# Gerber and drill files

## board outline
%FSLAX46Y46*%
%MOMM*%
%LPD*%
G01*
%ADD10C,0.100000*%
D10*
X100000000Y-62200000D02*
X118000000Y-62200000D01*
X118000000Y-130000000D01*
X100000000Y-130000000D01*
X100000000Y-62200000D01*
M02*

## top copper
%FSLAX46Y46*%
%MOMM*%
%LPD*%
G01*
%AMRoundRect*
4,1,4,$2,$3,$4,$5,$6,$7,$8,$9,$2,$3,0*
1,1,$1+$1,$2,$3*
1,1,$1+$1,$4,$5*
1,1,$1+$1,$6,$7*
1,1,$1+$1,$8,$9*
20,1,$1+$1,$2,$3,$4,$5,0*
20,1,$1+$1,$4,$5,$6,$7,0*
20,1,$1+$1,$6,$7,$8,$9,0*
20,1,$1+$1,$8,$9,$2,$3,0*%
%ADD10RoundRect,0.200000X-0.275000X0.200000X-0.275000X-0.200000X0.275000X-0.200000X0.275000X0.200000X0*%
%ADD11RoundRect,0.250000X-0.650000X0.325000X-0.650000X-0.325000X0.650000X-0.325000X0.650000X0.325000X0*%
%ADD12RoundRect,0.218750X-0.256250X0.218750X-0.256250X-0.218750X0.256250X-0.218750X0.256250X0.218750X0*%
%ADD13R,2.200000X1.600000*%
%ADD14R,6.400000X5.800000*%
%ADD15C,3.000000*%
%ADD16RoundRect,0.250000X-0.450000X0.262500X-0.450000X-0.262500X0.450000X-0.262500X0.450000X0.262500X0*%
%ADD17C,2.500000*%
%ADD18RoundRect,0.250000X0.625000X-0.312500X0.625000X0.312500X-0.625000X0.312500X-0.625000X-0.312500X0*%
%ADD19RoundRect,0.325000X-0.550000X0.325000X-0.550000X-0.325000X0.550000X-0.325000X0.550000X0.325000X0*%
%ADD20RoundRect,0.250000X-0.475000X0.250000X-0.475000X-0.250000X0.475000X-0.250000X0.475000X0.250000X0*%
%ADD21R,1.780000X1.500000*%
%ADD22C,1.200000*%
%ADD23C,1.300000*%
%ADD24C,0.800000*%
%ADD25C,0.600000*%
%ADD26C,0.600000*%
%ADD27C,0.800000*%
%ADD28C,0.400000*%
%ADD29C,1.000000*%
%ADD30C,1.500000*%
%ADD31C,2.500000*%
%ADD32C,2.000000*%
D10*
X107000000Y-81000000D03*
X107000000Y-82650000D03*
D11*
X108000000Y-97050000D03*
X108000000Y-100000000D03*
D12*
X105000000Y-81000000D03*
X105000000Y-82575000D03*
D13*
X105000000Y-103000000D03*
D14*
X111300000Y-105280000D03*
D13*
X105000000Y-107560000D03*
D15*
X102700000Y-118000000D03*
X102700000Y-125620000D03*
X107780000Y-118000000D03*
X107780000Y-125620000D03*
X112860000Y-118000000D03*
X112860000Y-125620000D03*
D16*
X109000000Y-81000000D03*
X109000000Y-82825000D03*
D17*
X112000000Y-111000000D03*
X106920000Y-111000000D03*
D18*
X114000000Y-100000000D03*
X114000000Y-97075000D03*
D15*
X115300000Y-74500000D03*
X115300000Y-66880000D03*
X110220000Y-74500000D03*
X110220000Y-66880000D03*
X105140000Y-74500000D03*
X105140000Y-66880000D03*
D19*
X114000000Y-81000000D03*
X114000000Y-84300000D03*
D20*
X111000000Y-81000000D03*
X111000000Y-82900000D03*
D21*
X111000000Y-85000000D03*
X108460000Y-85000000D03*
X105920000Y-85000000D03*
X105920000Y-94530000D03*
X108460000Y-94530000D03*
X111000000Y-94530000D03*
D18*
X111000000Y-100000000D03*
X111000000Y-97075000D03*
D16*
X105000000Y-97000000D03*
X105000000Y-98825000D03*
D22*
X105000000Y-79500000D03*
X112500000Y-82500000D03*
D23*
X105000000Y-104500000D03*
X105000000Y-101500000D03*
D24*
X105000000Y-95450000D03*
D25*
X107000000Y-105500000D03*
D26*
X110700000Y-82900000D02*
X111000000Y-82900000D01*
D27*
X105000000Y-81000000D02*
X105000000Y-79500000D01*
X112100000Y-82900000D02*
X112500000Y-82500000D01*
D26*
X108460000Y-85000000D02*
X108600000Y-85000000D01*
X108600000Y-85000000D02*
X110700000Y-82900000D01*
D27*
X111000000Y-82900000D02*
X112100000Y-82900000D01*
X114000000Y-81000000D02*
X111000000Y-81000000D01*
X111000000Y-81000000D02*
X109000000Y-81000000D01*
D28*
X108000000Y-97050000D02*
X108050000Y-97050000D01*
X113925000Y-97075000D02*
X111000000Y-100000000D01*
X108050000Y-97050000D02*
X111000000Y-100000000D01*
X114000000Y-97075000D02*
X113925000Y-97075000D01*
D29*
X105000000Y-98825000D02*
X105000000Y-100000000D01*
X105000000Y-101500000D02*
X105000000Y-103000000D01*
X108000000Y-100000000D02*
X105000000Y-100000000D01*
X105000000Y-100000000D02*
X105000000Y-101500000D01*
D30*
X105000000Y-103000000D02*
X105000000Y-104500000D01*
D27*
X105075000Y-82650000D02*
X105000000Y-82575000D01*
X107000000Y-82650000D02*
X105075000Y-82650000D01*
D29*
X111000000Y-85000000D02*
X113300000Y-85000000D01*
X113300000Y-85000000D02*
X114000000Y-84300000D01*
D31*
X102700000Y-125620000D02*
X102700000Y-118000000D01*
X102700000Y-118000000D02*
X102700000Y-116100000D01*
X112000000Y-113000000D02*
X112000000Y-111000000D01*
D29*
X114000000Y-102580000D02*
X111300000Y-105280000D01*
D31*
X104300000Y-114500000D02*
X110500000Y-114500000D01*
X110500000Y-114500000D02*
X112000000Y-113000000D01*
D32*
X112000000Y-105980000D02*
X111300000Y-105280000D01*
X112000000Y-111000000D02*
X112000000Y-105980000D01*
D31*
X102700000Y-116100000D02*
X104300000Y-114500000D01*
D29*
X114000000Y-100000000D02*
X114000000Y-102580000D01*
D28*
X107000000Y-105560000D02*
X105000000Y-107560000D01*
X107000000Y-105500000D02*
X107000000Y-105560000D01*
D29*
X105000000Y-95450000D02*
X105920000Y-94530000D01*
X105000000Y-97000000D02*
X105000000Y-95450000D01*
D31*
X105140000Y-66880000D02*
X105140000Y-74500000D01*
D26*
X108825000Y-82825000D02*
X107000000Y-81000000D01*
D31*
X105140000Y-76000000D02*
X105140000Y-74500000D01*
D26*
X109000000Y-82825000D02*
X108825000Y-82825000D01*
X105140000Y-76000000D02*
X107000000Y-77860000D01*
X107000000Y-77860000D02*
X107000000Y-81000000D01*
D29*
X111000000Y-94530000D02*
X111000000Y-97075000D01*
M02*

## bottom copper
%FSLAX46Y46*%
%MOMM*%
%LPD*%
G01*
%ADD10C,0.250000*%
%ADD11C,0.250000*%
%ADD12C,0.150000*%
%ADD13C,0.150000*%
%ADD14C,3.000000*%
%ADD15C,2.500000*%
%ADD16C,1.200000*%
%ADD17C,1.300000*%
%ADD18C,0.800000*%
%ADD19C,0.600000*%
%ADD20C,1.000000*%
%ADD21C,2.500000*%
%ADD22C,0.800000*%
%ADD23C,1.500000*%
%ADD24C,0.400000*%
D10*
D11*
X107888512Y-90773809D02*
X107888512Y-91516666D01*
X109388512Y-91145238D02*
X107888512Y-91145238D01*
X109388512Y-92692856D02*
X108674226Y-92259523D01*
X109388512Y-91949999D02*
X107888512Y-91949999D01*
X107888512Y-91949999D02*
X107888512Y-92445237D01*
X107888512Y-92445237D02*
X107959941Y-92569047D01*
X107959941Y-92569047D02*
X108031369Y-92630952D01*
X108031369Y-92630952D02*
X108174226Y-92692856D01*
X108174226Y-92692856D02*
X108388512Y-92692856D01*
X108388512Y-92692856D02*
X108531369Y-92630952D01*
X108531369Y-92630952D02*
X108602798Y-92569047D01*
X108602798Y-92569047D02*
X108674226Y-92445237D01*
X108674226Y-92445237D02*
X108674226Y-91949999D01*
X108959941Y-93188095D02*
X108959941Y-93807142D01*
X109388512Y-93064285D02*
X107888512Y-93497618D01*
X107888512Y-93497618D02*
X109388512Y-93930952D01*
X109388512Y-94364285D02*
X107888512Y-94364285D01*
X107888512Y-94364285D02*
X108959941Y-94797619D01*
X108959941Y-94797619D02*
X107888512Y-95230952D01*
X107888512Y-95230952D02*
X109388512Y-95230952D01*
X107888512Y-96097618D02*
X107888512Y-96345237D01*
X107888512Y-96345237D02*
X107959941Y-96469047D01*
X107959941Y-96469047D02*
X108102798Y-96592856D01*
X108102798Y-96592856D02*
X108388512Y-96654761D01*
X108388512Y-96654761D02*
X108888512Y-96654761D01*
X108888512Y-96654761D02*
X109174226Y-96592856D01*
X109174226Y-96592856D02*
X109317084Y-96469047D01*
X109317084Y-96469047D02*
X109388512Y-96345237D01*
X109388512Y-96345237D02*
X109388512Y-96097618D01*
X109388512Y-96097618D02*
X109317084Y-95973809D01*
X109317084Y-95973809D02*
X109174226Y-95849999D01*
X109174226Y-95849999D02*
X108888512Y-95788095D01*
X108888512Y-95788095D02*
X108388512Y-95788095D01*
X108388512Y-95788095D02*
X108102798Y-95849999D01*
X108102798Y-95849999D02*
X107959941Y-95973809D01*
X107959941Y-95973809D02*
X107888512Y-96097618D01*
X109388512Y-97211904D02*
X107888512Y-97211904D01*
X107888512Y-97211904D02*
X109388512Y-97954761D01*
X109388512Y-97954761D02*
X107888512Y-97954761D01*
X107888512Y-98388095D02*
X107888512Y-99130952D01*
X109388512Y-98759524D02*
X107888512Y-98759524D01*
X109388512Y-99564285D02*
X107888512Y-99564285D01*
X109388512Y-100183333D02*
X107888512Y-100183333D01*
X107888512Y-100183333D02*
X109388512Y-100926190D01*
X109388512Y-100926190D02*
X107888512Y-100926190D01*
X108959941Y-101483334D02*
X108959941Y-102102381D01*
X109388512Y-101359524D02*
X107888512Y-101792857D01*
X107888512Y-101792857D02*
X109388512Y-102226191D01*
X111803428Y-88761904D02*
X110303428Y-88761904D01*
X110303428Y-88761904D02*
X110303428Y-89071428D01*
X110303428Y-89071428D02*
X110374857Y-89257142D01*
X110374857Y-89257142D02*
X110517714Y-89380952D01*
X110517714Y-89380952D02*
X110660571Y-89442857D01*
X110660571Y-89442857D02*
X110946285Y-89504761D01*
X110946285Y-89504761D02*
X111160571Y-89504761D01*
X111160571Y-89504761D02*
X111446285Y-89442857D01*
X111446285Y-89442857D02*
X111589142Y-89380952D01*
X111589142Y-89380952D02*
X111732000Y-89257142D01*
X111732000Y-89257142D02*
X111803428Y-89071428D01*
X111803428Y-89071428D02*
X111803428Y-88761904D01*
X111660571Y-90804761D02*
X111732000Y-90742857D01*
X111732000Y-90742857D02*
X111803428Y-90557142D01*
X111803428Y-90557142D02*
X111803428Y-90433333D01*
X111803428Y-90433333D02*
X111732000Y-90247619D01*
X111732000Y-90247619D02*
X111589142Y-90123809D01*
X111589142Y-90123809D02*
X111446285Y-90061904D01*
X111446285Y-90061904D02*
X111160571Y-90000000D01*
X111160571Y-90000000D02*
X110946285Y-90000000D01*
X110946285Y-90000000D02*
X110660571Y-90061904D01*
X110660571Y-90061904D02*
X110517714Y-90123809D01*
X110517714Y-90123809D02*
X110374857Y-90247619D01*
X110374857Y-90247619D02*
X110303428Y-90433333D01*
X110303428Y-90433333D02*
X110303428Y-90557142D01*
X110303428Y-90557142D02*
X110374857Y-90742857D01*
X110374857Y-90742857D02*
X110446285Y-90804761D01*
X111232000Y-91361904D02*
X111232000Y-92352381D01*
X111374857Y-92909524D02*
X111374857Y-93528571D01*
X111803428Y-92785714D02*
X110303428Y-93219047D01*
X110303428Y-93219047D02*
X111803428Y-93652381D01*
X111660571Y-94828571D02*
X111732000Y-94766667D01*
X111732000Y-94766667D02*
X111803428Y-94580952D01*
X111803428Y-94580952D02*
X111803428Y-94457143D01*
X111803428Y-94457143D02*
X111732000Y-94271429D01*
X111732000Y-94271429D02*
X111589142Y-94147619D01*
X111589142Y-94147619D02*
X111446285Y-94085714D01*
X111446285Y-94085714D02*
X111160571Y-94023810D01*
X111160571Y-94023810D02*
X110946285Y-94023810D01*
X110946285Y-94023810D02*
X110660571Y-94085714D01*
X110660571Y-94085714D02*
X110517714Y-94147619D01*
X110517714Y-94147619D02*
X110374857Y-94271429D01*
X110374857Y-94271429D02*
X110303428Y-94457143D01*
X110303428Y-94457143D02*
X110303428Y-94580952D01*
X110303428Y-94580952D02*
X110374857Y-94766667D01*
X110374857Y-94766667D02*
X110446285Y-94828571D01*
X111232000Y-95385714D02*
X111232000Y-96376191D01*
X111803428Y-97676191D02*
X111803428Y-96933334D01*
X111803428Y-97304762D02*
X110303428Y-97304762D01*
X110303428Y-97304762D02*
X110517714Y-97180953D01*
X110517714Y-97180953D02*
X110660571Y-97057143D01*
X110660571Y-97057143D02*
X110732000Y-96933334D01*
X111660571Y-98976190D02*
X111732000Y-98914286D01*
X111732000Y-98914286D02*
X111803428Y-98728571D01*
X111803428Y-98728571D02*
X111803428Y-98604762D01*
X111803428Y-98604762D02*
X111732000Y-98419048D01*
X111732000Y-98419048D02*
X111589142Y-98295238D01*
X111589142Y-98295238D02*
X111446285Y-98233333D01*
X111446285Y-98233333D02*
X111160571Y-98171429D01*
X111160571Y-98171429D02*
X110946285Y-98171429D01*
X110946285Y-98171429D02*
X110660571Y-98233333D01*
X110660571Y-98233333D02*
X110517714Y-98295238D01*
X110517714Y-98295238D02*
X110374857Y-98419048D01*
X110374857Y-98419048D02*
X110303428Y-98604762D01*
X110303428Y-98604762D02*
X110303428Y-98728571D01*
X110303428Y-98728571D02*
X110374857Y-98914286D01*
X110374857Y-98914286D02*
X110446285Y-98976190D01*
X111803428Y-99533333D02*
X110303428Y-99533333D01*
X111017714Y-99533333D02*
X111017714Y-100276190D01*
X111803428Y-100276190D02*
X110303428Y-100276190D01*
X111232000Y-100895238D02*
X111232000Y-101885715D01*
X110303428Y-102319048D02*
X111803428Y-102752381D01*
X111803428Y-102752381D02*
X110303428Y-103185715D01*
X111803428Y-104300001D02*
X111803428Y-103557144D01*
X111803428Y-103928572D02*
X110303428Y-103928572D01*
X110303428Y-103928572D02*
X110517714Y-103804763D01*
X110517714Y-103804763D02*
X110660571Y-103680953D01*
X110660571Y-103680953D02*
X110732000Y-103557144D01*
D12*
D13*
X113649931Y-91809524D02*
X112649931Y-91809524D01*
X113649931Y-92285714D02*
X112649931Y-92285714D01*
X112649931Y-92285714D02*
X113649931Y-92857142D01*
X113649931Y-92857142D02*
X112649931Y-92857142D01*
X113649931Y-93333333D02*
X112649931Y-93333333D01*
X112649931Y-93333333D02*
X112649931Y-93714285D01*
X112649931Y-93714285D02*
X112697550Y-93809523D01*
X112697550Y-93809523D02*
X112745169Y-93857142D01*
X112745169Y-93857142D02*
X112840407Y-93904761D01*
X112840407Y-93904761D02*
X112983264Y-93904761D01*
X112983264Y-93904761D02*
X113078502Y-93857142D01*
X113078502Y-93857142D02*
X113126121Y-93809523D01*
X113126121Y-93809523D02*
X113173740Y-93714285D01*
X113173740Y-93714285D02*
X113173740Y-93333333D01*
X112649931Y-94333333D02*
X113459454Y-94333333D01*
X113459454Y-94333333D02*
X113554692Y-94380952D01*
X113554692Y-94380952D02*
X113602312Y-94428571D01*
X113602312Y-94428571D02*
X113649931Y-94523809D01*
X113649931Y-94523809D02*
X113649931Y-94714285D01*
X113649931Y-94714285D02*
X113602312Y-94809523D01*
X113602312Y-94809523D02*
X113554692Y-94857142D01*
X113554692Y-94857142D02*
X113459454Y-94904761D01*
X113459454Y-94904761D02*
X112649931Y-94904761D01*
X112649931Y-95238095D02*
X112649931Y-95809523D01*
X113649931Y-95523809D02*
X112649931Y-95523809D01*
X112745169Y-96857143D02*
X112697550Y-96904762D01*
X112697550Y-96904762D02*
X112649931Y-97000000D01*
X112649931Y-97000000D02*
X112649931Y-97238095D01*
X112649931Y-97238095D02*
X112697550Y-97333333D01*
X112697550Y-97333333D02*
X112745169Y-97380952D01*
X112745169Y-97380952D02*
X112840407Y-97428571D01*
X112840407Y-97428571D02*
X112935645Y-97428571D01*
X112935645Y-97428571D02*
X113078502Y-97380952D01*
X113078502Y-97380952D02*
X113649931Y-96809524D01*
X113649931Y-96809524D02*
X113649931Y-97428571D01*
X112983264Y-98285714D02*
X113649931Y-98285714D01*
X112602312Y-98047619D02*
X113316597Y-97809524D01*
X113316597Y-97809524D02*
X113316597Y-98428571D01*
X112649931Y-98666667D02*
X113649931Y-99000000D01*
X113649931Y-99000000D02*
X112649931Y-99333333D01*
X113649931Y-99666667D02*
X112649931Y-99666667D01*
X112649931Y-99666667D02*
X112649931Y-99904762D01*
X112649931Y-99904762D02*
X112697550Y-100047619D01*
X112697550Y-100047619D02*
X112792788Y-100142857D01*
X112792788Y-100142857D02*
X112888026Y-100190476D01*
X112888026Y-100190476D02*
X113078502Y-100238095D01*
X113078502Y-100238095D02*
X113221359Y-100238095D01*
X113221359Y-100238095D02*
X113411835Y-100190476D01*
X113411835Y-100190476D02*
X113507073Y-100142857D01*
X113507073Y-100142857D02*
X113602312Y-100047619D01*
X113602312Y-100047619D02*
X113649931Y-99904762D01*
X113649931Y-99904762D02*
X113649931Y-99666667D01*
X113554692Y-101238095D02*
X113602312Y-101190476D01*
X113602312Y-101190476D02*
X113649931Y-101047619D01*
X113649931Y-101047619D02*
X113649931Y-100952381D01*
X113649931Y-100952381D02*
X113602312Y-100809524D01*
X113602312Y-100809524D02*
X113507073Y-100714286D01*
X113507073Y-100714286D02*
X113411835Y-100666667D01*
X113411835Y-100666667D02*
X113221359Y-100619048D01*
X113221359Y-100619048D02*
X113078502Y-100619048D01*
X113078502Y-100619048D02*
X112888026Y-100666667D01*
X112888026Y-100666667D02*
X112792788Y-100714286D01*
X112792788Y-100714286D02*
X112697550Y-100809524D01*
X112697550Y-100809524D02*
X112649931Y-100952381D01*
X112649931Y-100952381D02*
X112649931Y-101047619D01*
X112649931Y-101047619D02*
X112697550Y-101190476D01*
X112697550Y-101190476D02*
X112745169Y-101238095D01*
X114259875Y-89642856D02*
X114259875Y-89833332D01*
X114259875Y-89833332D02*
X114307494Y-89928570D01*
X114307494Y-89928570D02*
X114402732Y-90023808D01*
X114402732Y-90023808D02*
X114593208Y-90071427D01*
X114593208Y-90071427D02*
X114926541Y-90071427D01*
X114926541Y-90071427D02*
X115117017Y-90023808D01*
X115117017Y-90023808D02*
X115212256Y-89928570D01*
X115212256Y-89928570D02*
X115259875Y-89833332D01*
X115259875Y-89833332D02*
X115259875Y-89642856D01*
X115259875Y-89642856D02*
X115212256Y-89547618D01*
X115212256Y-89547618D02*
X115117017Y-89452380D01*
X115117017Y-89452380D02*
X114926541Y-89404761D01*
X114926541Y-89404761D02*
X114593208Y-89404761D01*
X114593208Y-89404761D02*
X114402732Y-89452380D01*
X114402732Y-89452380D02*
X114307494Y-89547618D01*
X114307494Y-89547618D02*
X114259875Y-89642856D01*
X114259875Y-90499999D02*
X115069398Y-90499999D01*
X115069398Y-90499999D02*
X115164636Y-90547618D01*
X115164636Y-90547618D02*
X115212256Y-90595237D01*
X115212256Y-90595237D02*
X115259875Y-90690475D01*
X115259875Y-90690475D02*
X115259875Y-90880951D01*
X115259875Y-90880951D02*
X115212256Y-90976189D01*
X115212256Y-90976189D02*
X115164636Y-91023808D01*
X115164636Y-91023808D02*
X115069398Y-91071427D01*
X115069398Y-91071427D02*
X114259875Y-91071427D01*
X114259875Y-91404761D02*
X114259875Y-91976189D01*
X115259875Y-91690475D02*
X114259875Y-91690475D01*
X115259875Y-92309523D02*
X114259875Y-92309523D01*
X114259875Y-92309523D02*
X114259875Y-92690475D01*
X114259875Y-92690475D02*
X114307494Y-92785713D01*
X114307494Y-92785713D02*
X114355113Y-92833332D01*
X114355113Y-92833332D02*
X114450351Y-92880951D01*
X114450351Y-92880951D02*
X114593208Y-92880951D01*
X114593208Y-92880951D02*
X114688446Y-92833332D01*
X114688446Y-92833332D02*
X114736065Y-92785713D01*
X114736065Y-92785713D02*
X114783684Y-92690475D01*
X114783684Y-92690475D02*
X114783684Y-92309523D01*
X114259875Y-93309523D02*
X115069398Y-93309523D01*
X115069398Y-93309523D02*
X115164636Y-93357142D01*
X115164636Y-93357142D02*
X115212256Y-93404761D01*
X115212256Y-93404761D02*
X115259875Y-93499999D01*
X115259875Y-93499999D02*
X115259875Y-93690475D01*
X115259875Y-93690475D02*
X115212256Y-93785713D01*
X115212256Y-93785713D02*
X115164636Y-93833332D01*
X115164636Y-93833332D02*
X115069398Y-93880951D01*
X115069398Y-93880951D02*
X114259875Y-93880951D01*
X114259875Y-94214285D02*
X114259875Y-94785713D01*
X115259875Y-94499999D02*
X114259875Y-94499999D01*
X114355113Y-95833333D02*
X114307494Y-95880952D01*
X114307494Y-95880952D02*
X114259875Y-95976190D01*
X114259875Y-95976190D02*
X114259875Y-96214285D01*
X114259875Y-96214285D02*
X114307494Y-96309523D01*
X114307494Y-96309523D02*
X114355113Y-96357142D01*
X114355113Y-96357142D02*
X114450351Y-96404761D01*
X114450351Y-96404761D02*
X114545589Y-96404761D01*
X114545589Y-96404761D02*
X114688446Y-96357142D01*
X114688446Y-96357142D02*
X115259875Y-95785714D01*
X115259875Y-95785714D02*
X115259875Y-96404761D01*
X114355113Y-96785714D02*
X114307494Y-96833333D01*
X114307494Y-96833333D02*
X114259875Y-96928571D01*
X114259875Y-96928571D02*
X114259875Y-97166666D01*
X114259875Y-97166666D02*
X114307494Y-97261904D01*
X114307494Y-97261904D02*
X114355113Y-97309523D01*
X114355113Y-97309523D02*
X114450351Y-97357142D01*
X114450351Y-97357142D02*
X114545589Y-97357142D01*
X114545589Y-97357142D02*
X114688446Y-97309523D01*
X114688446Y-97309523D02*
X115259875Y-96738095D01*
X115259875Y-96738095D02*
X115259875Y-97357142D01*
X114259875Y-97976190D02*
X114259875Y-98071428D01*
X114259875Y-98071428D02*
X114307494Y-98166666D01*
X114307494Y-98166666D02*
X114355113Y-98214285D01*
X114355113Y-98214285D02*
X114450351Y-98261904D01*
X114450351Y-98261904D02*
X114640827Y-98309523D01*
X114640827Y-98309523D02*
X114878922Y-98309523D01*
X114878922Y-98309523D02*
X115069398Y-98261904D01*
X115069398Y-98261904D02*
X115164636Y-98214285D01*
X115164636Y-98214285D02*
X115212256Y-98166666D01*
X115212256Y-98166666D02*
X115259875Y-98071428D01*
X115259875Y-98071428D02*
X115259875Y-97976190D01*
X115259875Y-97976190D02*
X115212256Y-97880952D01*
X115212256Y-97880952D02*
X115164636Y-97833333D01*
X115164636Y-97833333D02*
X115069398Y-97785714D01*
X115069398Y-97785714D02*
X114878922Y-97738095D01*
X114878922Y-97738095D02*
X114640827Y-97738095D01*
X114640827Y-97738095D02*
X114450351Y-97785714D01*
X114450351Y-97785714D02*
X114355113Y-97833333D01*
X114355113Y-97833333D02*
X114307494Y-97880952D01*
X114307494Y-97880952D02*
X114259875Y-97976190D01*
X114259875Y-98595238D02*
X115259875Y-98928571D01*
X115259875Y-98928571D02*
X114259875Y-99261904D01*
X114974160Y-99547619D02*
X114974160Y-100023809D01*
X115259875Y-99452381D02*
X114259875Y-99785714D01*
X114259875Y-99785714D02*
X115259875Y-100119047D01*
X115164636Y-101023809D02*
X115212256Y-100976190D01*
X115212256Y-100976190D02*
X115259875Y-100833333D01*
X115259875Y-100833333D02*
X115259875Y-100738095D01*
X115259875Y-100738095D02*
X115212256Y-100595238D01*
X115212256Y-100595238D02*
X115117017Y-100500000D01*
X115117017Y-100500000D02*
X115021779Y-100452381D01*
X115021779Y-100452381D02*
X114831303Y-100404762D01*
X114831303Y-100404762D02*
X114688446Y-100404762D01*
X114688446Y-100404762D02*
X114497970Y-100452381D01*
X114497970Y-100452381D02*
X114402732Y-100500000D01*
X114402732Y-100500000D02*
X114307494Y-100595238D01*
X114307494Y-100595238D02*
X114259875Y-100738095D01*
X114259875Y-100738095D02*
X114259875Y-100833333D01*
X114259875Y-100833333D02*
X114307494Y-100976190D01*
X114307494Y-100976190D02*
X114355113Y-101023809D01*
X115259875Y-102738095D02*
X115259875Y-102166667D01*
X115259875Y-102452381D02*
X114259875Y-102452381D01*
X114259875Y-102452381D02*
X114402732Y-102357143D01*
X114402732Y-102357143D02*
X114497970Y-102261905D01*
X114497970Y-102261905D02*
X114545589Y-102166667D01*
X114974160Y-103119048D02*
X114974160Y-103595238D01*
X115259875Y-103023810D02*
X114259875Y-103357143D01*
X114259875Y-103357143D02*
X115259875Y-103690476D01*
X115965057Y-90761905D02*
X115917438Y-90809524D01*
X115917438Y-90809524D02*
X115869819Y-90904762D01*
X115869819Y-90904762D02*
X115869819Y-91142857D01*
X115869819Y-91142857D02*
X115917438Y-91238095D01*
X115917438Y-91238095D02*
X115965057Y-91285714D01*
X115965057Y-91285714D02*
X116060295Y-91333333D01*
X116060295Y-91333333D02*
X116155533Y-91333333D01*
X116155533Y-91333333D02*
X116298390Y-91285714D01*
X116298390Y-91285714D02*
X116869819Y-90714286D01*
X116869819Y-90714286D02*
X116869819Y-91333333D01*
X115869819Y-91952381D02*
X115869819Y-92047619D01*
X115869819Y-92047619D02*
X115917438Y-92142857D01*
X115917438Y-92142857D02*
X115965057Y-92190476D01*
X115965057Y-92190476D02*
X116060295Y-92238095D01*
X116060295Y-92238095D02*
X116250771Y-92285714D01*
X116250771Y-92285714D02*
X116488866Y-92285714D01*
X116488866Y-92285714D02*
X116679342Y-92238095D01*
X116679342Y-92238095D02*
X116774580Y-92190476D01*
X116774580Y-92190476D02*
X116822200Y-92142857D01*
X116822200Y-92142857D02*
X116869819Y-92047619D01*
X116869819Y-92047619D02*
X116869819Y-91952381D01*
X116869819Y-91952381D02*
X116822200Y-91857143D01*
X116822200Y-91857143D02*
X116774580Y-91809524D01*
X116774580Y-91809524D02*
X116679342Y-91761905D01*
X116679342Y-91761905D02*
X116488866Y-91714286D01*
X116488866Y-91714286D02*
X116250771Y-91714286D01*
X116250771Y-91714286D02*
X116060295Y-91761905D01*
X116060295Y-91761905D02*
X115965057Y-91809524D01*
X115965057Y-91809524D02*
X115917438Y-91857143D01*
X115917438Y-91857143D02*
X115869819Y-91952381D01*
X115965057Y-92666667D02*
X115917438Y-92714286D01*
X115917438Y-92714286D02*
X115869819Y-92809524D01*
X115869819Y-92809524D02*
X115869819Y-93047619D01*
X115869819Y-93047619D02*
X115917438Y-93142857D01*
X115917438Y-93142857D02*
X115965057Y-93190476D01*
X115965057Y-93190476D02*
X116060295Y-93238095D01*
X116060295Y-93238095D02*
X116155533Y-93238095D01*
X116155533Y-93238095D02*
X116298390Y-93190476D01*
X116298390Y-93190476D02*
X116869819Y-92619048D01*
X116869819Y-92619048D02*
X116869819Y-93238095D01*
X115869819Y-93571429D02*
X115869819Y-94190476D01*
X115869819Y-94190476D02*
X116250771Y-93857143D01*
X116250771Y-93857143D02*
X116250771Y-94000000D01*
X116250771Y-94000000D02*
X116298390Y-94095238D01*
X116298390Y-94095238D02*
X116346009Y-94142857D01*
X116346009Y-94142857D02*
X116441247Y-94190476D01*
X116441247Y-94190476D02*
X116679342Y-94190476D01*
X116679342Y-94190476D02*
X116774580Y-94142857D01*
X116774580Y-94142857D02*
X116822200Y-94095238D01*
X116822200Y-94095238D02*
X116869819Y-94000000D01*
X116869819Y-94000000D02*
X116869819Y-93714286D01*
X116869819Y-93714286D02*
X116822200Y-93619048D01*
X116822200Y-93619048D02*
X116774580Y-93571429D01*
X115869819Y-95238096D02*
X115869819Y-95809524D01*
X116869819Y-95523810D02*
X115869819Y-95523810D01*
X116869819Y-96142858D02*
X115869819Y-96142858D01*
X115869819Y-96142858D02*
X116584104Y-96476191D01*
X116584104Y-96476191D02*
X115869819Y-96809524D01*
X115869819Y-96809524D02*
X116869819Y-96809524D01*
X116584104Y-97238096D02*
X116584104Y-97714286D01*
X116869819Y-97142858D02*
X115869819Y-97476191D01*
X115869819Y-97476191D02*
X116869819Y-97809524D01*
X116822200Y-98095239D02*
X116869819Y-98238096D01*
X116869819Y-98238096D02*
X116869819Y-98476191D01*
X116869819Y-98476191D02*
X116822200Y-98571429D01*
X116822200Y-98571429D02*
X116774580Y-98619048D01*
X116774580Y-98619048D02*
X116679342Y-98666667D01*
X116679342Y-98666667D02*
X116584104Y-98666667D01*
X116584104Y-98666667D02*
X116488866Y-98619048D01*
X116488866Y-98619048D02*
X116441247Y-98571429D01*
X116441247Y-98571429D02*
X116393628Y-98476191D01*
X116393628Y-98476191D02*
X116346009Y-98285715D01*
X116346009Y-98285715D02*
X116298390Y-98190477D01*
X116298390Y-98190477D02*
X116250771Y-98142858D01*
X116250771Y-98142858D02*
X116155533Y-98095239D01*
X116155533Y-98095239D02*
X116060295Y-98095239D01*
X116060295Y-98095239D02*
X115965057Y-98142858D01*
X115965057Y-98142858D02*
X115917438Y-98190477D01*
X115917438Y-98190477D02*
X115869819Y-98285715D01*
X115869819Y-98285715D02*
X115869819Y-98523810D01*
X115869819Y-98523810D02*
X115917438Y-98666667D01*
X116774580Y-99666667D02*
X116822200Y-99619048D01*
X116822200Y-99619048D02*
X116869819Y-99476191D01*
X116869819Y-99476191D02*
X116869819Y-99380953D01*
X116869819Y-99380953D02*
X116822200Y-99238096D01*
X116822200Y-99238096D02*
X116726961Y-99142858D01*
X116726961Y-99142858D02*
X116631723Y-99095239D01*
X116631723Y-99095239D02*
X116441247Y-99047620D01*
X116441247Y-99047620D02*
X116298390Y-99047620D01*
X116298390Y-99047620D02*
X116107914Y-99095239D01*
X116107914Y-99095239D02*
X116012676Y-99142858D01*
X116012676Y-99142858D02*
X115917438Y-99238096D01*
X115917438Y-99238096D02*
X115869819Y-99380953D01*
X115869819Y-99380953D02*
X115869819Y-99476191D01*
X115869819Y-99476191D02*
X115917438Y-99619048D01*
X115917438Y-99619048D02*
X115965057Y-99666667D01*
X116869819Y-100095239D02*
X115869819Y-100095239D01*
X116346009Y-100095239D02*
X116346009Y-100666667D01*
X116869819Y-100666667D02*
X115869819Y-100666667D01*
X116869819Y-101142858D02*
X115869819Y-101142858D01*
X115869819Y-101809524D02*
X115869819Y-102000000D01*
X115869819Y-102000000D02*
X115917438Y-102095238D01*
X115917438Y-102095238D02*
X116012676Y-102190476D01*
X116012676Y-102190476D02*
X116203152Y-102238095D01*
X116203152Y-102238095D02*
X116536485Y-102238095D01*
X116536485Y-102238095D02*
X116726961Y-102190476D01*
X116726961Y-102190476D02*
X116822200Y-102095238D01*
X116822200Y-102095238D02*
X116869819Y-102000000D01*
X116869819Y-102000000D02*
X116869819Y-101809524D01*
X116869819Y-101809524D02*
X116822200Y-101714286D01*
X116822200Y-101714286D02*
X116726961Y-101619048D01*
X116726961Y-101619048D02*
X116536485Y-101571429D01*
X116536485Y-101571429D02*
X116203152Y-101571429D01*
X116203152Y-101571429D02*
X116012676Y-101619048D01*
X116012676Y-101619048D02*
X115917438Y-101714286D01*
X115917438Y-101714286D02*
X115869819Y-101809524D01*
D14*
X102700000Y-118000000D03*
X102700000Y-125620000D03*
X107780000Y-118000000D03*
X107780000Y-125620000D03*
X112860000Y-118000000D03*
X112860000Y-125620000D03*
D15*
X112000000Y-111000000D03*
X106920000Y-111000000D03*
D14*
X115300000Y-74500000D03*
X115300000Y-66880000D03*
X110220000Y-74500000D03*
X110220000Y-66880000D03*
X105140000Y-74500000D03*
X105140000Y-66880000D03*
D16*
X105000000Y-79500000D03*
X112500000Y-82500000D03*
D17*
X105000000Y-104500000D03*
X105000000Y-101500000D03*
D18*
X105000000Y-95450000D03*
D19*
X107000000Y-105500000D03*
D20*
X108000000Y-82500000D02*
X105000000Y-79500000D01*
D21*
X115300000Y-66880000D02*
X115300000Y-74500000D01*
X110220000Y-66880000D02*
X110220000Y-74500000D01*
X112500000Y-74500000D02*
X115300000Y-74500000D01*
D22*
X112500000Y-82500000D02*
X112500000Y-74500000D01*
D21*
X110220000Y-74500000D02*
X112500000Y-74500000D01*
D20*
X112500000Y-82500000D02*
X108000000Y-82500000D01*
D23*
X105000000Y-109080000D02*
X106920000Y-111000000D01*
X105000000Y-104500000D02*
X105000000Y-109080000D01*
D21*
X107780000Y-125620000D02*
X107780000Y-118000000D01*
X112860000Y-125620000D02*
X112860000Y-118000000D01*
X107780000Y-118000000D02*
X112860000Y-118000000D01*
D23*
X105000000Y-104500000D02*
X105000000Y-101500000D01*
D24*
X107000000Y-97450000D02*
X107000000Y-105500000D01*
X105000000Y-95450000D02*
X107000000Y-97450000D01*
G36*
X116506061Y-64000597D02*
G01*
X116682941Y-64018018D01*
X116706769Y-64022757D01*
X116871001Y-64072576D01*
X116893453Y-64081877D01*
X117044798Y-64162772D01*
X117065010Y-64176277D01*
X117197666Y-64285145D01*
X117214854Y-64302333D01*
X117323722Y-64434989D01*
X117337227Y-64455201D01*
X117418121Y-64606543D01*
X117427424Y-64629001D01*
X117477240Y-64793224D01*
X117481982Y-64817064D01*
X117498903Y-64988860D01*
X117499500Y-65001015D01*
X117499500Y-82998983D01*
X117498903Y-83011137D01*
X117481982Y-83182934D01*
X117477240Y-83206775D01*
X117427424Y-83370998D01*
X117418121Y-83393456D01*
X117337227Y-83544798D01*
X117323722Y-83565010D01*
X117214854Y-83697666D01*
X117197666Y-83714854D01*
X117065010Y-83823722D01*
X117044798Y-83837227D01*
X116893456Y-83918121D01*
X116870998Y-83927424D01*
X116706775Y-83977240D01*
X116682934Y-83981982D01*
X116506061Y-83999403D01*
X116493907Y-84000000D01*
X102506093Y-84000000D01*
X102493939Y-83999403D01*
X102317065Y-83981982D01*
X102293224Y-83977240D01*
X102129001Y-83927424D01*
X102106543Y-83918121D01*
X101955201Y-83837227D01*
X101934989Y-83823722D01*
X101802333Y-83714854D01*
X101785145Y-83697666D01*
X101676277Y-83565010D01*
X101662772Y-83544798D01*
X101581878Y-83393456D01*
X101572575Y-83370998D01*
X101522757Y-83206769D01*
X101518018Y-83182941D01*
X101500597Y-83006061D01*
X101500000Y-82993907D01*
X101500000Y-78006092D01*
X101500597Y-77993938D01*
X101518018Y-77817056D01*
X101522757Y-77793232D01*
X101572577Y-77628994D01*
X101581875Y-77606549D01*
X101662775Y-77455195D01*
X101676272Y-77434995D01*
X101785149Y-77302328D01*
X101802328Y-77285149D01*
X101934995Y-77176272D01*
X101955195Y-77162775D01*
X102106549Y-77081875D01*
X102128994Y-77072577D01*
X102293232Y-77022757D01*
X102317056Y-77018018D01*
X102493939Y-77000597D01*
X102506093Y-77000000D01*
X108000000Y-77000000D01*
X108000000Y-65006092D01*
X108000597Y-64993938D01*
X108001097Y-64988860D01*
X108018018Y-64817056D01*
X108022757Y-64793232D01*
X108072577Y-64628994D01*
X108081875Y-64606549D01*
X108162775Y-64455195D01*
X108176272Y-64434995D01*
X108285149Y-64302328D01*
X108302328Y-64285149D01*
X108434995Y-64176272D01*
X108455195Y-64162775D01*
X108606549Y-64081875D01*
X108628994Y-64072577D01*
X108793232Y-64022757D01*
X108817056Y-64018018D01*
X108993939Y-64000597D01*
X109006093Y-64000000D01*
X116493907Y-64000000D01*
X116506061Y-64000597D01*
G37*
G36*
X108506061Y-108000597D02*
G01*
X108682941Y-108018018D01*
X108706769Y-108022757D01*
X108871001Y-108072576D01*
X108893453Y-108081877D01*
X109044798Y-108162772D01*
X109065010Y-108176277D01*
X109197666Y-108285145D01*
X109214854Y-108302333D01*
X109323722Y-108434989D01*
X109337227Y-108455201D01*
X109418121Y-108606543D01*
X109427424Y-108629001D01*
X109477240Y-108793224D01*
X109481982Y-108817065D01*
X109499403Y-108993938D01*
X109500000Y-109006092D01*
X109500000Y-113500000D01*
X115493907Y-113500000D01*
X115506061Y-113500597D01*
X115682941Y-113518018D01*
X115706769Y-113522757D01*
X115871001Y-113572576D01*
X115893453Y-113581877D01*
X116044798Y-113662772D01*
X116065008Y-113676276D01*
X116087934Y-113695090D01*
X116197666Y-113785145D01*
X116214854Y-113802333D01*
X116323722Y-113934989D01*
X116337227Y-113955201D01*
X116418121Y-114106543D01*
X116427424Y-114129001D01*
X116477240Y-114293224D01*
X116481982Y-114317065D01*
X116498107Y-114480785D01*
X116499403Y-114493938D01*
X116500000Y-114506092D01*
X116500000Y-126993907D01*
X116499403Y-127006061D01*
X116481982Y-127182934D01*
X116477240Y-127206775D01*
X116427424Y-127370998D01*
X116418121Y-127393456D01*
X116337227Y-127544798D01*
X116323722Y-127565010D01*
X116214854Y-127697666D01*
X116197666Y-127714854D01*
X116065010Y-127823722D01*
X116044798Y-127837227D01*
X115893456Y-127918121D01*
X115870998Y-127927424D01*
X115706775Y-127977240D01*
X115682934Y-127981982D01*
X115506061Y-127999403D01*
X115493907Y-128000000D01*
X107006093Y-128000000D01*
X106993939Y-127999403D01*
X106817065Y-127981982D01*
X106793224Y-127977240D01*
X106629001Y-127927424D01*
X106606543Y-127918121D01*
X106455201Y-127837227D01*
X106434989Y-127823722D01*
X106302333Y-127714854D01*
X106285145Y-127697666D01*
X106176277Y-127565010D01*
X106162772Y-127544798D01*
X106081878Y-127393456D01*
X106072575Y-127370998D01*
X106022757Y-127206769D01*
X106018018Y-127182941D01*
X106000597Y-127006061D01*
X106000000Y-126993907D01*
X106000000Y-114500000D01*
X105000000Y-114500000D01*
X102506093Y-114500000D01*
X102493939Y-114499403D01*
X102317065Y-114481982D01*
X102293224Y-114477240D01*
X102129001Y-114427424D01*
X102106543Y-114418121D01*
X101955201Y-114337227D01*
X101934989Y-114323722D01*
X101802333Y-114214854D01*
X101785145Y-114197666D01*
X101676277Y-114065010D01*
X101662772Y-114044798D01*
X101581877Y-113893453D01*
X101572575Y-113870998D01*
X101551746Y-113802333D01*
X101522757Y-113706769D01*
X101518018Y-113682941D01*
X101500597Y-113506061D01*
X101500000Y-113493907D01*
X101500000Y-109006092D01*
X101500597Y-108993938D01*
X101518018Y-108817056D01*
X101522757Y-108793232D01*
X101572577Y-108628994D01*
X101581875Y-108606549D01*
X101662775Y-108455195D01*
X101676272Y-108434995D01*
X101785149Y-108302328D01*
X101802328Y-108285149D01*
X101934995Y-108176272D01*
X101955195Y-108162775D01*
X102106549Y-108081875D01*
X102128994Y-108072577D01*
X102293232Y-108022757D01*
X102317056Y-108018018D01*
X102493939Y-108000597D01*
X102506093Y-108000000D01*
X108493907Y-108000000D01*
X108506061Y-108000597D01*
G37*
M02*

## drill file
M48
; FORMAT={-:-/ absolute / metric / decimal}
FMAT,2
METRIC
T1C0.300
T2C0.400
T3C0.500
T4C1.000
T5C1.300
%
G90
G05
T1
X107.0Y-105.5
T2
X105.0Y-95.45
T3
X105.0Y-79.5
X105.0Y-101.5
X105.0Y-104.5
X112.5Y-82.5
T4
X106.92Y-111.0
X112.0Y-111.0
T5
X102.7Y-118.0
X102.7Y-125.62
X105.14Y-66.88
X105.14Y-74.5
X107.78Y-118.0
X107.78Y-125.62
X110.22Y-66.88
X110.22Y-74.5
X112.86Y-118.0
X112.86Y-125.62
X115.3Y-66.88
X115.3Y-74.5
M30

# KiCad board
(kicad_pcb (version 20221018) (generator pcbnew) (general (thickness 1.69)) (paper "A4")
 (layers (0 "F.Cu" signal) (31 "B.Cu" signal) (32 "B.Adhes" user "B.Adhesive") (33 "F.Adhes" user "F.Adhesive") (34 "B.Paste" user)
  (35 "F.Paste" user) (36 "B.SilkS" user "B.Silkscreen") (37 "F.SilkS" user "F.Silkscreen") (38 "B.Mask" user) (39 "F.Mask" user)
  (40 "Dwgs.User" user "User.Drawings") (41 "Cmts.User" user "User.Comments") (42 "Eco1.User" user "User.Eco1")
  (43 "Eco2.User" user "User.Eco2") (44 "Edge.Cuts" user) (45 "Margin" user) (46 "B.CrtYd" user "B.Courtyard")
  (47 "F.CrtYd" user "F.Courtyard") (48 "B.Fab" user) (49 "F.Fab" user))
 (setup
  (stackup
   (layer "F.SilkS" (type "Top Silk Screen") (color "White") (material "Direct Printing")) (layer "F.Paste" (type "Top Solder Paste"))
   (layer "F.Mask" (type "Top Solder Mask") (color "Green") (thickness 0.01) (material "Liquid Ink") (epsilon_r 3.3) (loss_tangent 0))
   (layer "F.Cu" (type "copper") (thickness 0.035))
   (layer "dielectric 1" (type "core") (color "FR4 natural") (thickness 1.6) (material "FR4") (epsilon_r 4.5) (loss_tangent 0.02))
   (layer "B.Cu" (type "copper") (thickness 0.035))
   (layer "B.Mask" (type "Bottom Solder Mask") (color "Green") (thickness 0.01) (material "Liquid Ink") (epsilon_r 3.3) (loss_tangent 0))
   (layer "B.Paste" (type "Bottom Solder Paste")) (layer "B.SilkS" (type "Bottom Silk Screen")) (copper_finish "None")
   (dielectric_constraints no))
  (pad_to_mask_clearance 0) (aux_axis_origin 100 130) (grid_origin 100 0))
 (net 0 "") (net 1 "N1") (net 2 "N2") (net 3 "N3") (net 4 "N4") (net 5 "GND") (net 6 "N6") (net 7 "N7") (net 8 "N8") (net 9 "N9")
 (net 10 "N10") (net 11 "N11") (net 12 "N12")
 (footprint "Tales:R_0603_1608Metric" (layer "F.Cu") (at 107 81.825 -90)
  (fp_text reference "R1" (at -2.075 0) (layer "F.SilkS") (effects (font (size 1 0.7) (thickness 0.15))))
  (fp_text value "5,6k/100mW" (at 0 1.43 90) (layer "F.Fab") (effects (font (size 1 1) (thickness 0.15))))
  (pad "1" smd roundrect (at -0.825 0 270) (size 0.8 0.95) (layers "F.Cu" "F.Paste" "F.Mask") (roundrect_rratio 0.25) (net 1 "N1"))
  (pad "2" smd roundrect (at 0.825 0 270) (size 0.8 0.95) (layers "F.Cu" "F.Paste" "F.Mask") (roundrect_rratio 0.25) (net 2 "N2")))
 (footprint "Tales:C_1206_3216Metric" (layer "F.Cu") (at 108 98.525 -90)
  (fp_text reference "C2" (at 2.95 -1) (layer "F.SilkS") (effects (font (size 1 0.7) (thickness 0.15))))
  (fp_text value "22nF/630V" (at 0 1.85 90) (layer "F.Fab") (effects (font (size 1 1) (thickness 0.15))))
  (pad "1" smd roundrect (at -1.475 0 270) (size 1.15 1.8) (layers "F.Cu" "F.Paste" "F.Mask") (roundrect_rratio 0.2173913043) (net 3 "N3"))
  (pad "2" smd roundrect (at 1.475 0 270) (size 1.15 1.8) (layers "F.Cu" "F.Paste" "F.Mask") (roundrect_rratio 0.2173913043) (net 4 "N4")))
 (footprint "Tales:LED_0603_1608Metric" (layer "F.Cu") (at 105 81.7875 -90)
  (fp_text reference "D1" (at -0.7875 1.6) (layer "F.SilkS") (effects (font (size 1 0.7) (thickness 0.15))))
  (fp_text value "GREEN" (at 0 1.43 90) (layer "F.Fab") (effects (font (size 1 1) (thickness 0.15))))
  (pad "1" smd roundrect (at -0.7875 0 270) (size 0.875 0.95) (layers "F.Cu" "F.Paste" "F.Mask") (roundrect_rratio 0.25) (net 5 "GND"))
  (pad "2" smd roundrect (at 0.7875 0 270) (size 0.875 0.95) (layers "F.Cu" "F.Paste" "F.Mask") (roundrect_rratio 0.25) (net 2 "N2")))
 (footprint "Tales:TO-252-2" (layer "F.Cu") (at 109.2 105.28)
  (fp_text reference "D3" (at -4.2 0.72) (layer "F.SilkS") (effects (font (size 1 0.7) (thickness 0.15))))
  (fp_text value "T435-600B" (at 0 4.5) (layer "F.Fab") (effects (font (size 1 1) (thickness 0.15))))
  (pad "" smd rect (at 0.425 -1.525) (size 3.05 2.75) (layers "F.Paste"))
  (pad "" smd rect (at 0.425 1.525) (size 3.05 2.75) (layers "F.Paste"))
  (pad "" smd rect (at 3.775 -1.525) (size 3.05 2.75) (layers "F.Paste"))
  (pad "" smd rect (at 3.775 1.525) (size 3.05 2.75) (layers "F.Paste"))
  (pad "1" smd rect (at -4.2 -2.28) (size 2.2 1.6) (layers "F.Cu" "F.Paste" "F.Mask") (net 4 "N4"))
  (pad "2" smd rect (at 2.1 0) (size 6.4 5.8) (layers "F.Cu" "F.Mask") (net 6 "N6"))
  (pad "3" smd rect (at -4.2 2.28) (size 2.2 1.6) (layers "F.Cu" "F.Paste" "F.Mask") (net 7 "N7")))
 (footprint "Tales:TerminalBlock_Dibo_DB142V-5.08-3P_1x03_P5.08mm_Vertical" (layer "F.Cu") (at 102.7 125.62)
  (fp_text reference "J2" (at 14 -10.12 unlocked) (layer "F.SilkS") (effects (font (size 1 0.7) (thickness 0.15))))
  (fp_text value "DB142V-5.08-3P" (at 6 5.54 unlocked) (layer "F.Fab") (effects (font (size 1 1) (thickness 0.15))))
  (pad "1" thru_hole circle (at 0 -7.62 180) (size 3 3) (drill 1.3) (layers "*.Cu" "*.Mask") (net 6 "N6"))
  (pad "1" thru_hole circle (at 0 0 180) (size 3 3) (drill 1.3) (layers "*.Cu" "*.Mask") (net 6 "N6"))
  (pad "2" thru_hole circle (at 5.08 -7.62 180) (size 3 3) (drill 1.3) (layers "*.Cu" "*.Mask") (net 4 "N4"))
  (pad "2" thru_hole circle (at 5.08 0 180) (size 3 3) (drill 1.3) (layers "*.Cu" "*.Mask") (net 4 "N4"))
  (pad "3" thru_hole circle (at 10.16 -7.62 180) (size 3 3) (drill 1.3) (layers "*.Cu" "*.Mask") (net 4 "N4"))
  (pad "3" thru_hole circle (at 10.16 0 180) (size 3 3) (drill 1.3) (layers "*.Cu" "*.Mask") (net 4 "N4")))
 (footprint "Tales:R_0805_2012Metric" (layer "F.Cu") (at 109 81.9125 -90)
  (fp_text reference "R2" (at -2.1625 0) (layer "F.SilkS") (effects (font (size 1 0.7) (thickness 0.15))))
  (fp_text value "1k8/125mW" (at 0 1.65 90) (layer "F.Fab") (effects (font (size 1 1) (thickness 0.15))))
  (pad "1" smd roundrect (at -0.9125 0 270) (size 1.025 1.4) (layers "F.Cu" "F.Paste" "F.Mask") (roundrect_rratio 0.243902439) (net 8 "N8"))
  (pad "2" smd roundrect (at 0.9125 0 270) (size 1.025 1.4) (layers "F.Cu" "F.Paste" "F.Mask") (roundrect_rratio 0.243902439) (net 1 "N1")))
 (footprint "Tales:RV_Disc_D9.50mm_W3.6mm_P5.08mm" (layer "F.Cu") (at 112 111 180)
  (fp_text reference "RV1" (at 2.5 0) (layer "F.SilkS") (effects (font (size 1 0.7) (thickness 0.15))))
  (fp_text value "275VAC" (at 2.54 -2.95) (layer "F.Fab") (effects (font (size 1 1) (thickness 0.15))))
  (pad "1" thru_hole circle (at 0 0 180) (size 2.5 2.5) (drill 1) (layers "*.Cu" "*.Mask") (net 6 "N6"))
  (pad "2" thru_hole circle (at 5.08 0 180) (size 2.5 2.5) (drill 1) (layers "*.Cu" "*.Mask") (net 4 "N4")))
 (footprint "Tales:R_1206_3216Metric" (layer "F.Cu") (at 114 98.5375 90)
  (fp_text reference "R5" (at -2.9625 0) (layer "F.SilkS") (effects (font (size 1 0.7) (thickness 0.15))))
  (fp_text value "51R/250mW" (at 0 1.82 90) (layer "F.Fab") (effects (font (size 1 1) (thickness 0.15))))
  (pad "1" smd roundrect (at -1.4625 0 90) (size 1.125 1.75) (layers "F.Cu" "F.Paste" "F.Mask") (roundrect_rratio 0.2222222222) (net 6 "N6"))
  (pad "2" smd roundrect (at 1.4625 0 90) (size 1.125 1.75) (layers "F.Cu" "F.Paste" "F.Mask") (roundrect_rratio 0.2222222222) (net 3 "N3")))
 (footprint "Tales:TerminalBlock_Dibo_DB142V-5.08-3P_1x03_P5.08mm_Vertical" (layer "F.Cu") (at 115.3 66.88 180)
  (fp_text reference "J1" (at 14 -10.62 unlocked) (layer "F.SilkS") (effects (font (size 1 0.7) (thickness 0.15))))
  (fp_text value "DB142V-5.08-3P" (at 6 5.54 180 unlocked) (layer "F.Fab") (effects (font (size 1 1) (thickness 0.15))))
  (pad "1" thru_hole circle (at 0 -7.62) (size 3 3) (drill 1.3) (layers "*.Cu" "*.Mask") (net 5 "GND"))
  (pad "1" thru_hole circle (at 0 0) (size 3 3) (drill 1.3) (layers "*.Cu" "*.Mask") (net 5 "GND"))
  (pad "2" thru_hole circle (at 5.08 -7.62) (size 3 3) (drill 1.3) (layers "*.Cu" "*.Mask") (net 5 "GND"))
  (pad "2" thru_hole circle (at 5.08 0) (size 3 3) (drill 1.3) (layers "*.Cu" "*.Mask") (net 5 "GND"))
  (pad "3" thru_hole circle (at 10.16 -7.62) (size 3 3) (drill 1.3) (layers "*.Cu" "*.Mask") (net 1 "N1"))
  (pad "3" thru_hole circle (at 10.16 0) (size 3 3) (drill 1.3) (layers "*.Cu" "*.Mask") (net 1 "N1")))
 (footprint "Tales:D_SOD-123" (layer "F.Cu") (at 114 82.65 -90)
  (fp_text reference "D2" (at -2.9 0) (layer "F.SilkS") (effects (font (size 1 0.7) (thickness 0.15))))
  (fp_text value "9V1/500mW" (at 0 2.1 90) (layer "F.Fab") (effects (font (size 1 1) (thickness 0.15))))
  (pad "1" smd roundrect (at -1.65 0 270) (size 1.3 1.75) (layers "F.Cu" "F.Paste" "F.Mask") (roundrect_rratio 0.25) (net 8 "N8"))
  (pad "2" smd roundrect (at 1.65 0 270) (size 1.3 1.75) (layers "F.Cu" "F.Paste" "F.Mask") (roundrect_rratio 0.25) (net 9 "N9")))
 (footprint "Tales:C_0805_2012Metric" (layer "F.Cu") (at 111 81.95 -90)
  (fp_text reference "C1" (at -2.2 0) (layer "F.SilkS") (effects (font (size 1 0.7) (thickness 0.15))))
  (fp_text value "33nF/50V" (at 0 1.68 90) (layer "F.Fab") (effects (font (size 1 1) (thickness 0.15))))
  (pad "1" smd roundrect (at -0.95 0 270) (size 1 1.45) (layers "F.Cu" "F.Paste" "F.Mask") (roundrect_rratio 0.25) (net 8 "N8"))
  (pad "2" smd roundrect (at 0.95 0 270) (size 1 1.45) (layers "F.Cu" "F.Paste" "F.Mask") (roundrect_rratio 0.25) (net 5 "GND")))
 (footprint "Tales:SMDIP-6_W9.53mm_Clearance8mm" (layer "F.Cu") (at 108.46 89.765 -90)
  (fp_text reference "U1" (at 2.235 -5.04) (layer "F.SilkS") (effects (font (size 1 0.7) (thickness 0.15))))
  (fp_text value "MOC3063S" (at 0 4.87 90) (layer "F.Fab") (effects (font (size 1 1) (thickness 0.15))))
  (pad "1" smd rect (at -4.765 -2.54 270) (size 1.5 1.78) (layers "F.Cu" "F.Paste" "F.Mask") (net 9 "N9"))
  (pad "2" smd rect (at -4.765 0 270) (size 1.5 1.78) (layers "F.Cu" "F.Paste" "F.Mask") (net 5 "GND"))
  (pad "3" smd rect (at -4.765 2.54 270) (size 1.5 1.78) (layers "F.Cu" "F.Paste" "F.Mask") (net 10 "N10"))
  (pad "4" smd rect (at 4.765 2.54 270) (size 1.5 1.78) (layers "F.Cu" "F.Paste" "F.Mask") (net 7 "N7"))
  (pad "5" smd rect (at 4.765 0 270) (size 1.5 1.78) (layers "F.Cu" "F.Paste" "F.Mask") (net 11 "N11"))
  (pad "6" smd rect (at 4.765 -2.54 270) (size 1.5 1.78) (layers "F.Cu" "F.Paste" "F.Mask") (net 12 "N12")))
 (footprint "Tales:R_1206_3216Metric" (layer "F.Cu") (at 111 98.5375 90)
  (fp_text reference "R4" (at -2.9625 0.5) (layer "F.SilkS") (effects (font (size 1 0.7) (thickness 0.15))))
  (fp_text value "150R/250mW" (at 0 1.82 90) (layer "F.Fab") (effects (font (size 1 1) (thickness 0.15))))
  (pad "1" smd roundrect (at -1.4625 0 90) (size 1.125 1.75) (layers "F.Cu" "F.Paste" "F.Mask") (roundrect_rratio 0.2222222222) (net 3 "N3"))
  (pad "2" smd roundrect (at 1.4625 0 90) (size 1.125 1.75) (layers "F.Cu" "F.Paste" "F.Mask") (roundrect_rratio 0.2222222222)
   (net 12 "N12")))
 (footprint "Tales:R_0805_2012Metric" (layer "F.Cu") (at 105 97.9125 -90)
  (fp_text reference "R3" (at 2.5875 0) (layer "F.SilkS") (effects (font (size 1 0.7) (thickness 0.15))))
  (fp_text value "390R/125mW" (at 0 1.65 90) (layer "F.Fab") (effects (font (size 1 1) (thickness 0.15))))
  (pad "1" smd roundrect (at -0.9125 0 270) (size 1.025 1.4) (layers "F.Cu" "F.Paste" "F.Mask") (roundrect_rratio 0.243902439) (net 7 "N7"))
  (pad "2" smd roundrect (at 0.9125 0 270) (size 1.025 1.4) (layers "F.Cu" "F.Paste" "F.Mask") (roundrect_rratio 0.243902439) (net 4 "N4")))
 (gr_rect (start 100 62.2) (end 118 130) (stroke (width 0.1) (type solid)) (fill none) (layer "Edge.Cuts"))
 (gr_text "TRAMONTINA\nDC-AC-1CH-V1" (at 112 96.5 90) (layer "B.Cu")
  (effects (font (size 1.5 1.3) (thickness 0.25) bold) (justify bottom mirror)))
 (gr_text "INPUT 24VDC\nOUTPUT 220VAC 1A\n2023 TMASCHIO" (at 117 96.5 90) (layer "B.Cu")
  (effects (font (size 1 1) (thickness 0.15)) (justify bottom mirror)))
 (segment (start 110.7 82.9) (end 111 82.9) (width 0.6) (layer "F.Cu") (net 5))
 (segment (start 105 81) (end 105 79.5) (width 0.8) (layer "F.Cu") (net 5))
 (segment (start 112.1 82.9) (end 112.5 82.5) (width 0.8) (layer "F.Cu") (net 5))
 (segment (start 108.46 85) (end 108.6 85) (width 0.6) (layer "F.Cu") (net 5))
 (segment (start 108.6 85) (end 110.7 82.9) (width 0.6) (layer "F.Cu") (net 5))
 (segment (start 111 82.9) (end 112.1 82.9) (width 0.8) (layer "F.Cu") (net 5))
 (via (at 105 79.5) (size 1.2) (drill 0.5) (layers "F.Cu" "B.Cu") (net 5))
 (via (at 112.5 82.5) (size 1.2) (drill 0.5) (layers "F.Cu" "B.Cu") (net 5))
 (segment (start 108 82.5) (end 105 79.5) (width 1) (layer "B.Cu") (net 5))
 (segment (start 115.3 66.88) (end 115.3 74.5) (width 2.5) (layer "B.Cu") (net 5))
 (segment (start 110.22 66.88) (end 110.22 74.5) (width 2.5) (layer "B.Cu") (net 5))
 (segment (start 112.5 74.5) (end 115.3 74.5) (width 2.5) (layer "B.Cu") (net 5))
 (segment (start 112.5 82.5) (end 112.5 74.5) (width 0.8) (layer "B.Cu") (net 5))
 (segment (start 110.22 74.5) (end 112.5 74.5) (width 2.5) (layer "B.Cu") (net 5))
 (segment (start 112.5 82.5) (end 108 82.5) (width 1) (layer "B.Cu") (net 5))
 (segment (start 114 81) (end 111 81) (width 0.8) (layer "F.Cu") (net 8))
 (segment (start 111 81) (end 109 81) (width 0.8) (layer "F.Cu") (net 8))
 (segment (start 108 97.05) (end 108.05 97.05) (width 0.4) (layer "F.Cu") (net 3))
 (segment (start 113.925 97.075) (end 111 100) (width 0.4) (layer "F.Cu") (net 3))
 (segment (start 108.05 97.05) (end 111 100) (width 0.4) (layer "F.Cu") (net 3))
 (segment (start 114 97.075) (end 113.925 97.075) (width 0.4) (layer "F.Cu") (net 3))
 (segment (start 105 98.825) (end 105 100) (width 1) (layer "F.Cu") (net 4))
 (segment (start 105 101.5) (end 105 103) (width 1) (layer "F.Cu") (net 4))
 (segment (start 108 100) (end 105 100) (width 1) (layer "F.Cu") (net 4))
 (segment (start 105 100) (end 105 101.5) (width 1) (layer "F.Cu") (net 4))
 (segment (start 105 103) (end 105 104.5) (width 1.5) (layer "F.Cu") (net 4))
 (via (at 105 104.5) (size 1.3) (drill 0.5) (layers "F.Cu" "B.Cu") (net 4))
 (via (at 105 101.5) (size 1.3) (drill 0.5) (layers "F.Cu" "B.Cu") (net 4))
 (segment (start 105 109.08) (end 106.92 111) (width 1.5) (layer "B.Cu") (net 4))
 (segment (start 105 104.5) (end 105 109.08) (width 1.5) (layer "B.Cu") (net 4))
 (segment (start 107.78 125.62) (end 107.78 118) (width 2.5) (layer "B.Cu") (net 4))
 (segment (start 112.86 125.62) (end 112.86 118) (width 2.5) (layer "B.Cu") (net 4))
 (segment (start 107.78 118) (end 112.86 118) (width 2.5) (layer "B.Cu") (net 4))
 (segment (start 105 104.5) (end 105 101.5) (width 1.5) (layer "B.Cu") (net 4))
 (segment (start 105.075 82.65) (end 105 82.575) (width 0.8) (layer "F.Cu") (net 2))
 (segment (start 107 82.65) (end 105.075 82.65) (width 0.8) (layer "F.Cu") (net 2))
 (segment (start 111 85) (end 113.3 85) (width 1) (layer "F.Cu") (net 9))
 (segment (start 113.3 85) (end 114 84.3) (width 1) (layer "F.Cu") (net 9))
 (segment (start 102.7 125.62) (end 102.7 118) (width 2.5) (layer "F.Cu") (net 6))
 (segment (start 102.7 118) (end 102.7 116.1) (width 2.5) (layer "F.Cu") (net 6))
 (segment (start 112 113) (end 112 111) (width 2.5) (layer "F.Cu") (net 6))
 (segment (start 114 102.58) (end 111.3 105.28) (width 1) (layer "F.Cu") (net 6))
 (segment (start 104.3 114.5) (end 110.5 114.5) (width 2.5) (layer "F.Cu") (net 6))
 (segment (start 110.5 114.5) (end 112 113) (width 2.5) (layer "F.Cu") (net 6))
 (segment (start 112 105.98) (end 111.3 105.28) (width 2) (layer "F.Cu") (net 6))
 (segment (start 112 111) (end 112 105.98) (width 2) (layer "F.Cu") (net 6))
 (segment (start 102.7 116.1) (end 104.3 114.5) (width 2.5) (layer "F.Cu") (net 6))
 (segment (start 114 100) (end 114 102.58) (width 1) (layer "F.Cu") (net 6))
 (segment (start 107 105.56) (end 105 107.56) (width 0.4) (layer "F.Cu") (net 7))
 (segment (start 107 105.5) (end 107 105.56) (width 0.4) (layer "F.Cu") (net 7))
 (segment (start 105 95.45) (end 105.92 94.53) (width 1) (layer "F.Cu") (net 7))
 (segment (start 105 97) (end 105 95.45) (width 1) (layer "F.Cu") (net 7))
 (via (at 105 95.45) (size 0.8) (drill 0.4) (layers "F.Cu" "B.Cu") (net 7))
 (via (at 107 105.5) (size 0.6) (drill 0.3) (layers "F.Cu" "B.Cu") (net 7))
 (segment (start 107 97.45) (end 107 105.5) (width 0.4) (layer "B.Cu") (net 7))
 (segment (start 105 95.45) (end 107 97.45) (width 0.4) (layer "B.Cu") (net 7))
 (segment (start 105.14 66.88) (end 105.14 74.5) (width 2.5) (layer "F.Cu") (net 1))
 (segment (start 108.825 82.825) (end 107 81) (width 0.6) (layer "F.Cu") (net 1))
 (segment (start 105.14 76) (end 105.14 74.5) (width 2.5) (layer "F.Cu") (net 1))
 (segment (start 109 82.825) (end 108.825 82.825) (width 0.6) (layer "F.Cu") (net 1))
 (segment (start 105.14 76) (end 107 77.86) (width 0.6) (layer "F.Cu") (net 1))
 (segment (start 107 77.86) (end 107 81) (width 0.6) (layer "F.Cu") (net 1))
 (segment (start 111 94.53) (end 111 97.075) (width 1) (layer "F.Cu") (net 12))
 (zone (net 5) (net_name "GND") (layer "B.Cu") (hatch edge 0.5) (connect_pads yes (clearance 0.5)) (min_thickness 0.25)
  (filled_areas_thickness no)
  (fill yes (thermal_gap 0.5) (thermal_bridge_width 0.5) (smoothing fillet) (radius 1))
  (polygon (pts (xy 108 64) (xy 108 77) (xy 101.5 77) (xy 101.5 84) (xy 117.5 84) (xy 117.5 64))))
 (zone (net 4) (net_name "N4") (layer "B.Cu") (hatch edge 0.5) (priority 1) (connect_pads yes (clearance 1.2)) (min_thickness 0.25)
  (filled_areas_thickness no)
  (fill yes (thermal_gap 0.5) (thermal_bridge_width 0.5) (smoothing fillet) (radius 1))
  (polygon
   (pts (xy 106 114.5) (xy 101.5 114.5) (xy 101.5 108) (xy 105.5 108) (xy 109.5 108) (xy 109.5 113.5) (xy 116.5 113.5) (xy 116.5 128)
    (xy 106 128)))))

